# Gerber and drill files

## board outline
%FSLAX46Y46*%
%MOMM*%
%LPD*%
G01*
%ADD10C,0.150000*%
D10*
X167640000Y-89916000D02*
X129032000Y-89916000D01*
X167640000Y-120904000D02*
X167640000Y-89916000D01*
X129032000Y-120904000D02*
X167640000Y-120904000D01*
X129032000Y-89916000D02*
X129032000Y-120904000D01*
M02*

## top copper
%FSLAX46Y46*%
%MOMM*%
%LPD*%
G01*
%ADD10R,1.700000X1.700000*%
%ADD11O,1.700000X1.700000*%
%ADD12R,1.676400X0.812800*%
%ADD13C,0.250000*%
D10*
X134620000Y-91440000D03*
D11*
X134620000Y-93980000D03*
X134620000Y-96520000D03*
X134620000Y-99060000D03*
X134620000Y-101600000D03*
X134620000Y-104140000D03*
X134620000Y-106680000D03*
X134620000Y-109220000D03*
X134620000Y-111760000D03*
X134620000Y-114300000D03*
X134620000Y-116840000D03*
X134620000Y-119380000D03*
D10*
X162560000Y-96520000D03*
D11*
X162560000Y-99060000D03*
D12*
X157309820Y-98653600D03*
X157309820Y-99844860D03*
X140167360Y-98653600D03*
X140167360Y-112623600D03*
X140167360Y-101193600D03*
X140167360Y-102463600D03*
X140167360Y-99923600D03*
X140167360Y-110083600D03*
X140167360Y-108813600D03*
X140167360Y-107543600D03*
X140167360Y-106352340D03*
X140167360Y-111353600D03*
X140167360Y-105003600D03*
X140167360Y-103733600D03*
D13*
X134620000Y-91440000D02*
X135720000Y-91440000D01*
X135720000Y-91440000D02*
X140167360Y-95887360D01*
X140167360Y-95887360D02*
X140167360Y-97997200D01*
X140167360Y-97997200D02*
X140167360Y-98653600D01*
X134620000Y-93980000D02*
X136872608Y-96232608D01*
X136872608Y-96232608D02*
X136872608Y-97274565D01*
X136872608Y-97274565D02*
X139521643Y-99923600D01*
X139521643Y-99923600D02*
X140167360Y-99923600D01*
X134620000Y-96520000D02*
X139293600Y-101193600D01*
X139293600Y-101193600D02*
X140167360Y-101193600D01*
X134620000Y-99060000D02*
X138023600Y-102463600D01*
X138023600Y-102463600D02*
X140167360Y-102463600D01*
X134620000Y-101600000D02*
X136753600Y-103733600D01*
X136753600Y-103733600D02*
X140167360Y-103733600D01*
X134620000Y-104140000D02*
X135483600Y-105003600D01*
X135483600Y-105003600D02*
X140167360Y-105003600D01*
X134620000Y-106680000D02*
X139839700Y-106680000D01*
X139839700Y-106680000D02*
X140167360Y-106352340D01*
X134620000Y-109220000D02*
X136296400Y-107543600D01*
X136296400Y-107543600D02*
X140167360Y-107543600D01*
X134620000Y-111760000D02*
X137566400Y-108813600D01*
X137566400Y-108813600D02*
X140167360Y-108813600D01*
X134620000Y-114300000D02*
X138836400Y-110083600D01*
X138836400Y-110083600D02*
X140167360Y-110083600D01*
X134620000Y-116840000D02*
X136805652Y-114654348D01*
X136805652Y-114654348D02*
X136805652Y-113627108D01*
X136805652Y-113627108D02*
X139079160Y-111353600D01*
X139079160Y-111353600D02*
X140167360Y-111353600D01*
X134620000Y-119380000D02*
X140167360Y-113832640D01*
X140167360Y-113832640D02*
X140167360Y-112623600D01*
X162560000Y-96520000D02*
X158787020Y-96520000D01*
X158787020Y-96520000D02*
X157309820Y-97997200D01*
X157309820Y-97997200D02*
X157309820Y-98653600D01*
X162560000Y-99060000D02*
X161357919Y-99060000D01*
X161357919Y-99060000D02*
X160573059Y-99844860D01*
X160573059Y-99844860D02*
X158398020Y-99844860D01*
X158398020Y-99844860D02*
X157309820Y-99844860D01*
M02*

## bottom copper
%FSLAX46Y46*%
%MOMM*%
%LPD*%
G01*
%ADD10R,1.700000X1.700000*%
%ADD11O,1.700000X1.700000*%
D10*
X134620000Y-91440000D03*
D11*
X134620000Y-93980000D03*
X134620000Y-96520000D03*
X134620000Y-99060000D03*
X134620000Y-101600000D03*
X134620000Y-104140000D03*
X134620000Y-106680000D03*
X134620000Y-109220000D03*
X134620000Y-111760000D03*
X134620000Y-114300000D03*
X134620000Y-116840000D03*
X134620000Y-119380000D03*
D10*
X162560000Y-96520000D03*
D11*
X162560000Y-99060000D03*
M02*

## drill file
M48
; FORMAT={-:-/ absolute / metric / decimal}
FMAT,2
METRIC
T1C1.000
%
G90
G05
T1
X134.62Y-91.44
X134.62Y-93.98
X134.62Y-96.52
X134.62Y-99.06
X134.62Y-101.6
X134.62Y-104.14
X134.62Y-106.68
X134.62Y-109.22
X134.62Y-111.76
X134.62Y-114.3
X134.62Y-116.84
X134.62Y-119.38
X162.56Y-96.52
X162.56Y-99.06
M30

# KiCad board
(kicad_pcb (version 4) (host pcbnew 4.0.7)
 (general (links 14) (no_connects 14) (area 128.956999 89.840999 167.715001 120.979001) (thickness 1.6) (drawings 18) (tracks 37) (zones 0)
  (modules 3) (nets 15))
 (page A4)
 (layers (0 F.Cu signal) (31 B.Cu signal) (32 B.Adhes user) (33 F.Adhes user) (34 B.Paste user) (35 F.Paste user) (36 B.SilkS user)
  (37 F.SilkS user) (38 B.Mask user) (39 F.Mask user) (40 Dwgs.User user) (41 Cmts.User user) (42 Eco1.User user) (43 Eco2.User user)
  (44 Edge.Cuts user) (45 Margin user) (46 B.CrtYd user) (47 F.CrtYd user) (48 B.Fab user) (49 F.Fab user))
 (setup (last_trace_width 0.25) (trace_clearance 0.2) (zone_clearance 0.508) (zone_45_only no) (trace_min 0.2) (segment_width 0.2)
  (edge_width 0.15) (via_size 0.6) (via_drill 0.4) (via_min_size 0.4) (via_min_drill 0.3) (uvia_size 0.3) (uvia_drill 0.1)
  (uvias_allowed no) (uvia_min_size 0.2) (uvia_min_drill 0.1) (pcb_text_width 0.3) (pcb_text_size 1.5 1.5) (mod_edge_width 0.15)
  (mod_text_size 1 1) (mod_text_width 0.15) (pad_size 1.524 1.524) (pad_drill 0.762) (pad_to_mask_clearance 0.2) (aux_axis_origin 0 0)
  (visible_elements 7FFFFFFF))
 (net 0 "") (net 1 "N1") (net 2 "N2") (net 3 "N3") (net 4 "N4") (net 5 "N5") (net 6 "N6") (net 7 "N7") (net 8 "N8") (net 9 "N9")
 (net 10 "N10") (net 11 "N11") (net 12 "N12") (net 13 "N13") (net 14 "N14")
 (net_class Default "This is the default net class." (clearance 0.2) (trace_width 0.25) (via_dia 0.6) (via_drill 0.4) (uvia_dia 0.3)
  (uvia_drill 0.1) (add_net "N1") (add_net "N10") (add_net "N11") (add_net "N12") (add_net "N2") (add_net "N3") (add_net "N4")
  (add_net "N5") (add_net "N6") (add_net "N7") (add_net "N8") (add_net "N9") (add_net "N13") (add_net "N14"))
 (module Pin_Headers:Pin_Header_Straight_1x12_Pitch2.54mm (layer F.Cu) (at 134.62 91.44)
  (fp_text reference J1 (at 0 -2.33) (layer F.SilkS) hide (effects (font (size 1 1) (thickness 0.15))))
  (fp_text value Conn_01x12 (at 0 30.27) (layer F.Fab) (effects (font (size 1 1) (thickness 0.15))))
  (pad 1 thru_hole rect (at 0 0) (size 1.7 1.7) (drill 1) (layers *.Cu *.Mask) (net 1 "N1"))
  (pad 2 thru_hole oval (at 0 2.54) (size 1.7 1.7) (drill 1) (layers *.Cu *.Mask) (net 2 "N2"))
  (pad 3 thru_hole oval (at 0 5.08) (size 1.7 1.7) (drill 1) (layers *.Cu *.Mask) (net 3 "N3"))
  (pad 4 thru_hole oval (at 0 7.62) (size 1.7 1.7) (drill 1) (layers *.Cu *.Mask) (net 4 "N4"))
  (pad 5 thru_hole oval (at 0 10.16) (size 1.7 1.7) (drill 1) (layers *.Cu *.Mask) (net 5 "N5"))
  (pad 6 thru_hole oval (at 0 12.7) (size 1.7 1.7) (drill 1) (layers *.Cu *.Mask) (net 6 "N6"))
  (pad 7 thru_hole oval (at 0 15.24) (size 1.7 1.7) (drill 1) (layers *.Cu *.Mask) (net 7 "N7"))
  (pad 8 thru_hole oval (at 0 17.78) (size 1.7 1.7) (drill 1) (layers *.Cu *.Mask) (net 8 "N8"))
  (pad 9 thru_hole oval (at 0 20.32) (size 1.7 1.7) (drill 1) (layers *.Cu *.Mask) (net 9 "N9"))
  (pad 10 thru_hole oval (at 0 22.86) (size 1.7 1.7) (drill 1) (layers *.Cu *.Mask) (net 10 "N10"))
  (pad 11 thru_hole oval (at 0 25.4) (size 1.7 1.7) (drill 1) (layers *.Cu *.Mask) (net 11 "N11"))
  (pad 12 thru_hole oval (at 0 27.94) (size 1.7 1.7) (drill 1) (layers *.Cu *.Mask) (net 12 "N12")))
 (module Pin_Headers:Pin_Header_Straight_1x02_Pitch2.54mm (layer F.Cu) (at 162.56 96.52)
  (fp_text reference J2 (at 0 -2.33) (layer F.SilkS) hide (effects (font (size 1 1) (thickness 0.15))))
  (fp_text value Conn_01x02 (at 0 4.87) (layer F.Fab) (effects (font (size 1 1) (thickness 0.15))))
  (pad 1 thru_hole rect (at 0 0) (size 1.7 1.7) (drill 1) (layers *.Cu *.Mask) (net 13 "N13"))
  (pad 2 thru_hole oval (at 0 2.54) (size 1.7 1.7) (drill 1) (layers *.Cu *.Mask) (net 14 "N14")))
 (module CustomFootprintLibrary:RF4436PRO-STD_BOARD (layer F.Cu) (at 148.5011 105.0036)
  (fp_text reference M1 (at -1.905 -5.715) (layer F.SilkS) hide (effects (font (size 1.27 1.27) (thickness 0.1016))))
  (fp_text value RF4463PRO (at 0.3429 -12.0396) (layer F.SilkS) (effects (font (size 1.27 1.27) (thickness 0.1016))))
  (pad 13 smd rect (at 8.80872 -6.35) (size 1.6764 0.8128) (layers F.Cu F.Paste F.Mask) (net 13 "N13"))
  (pad 14 smd rect (at 8.80872 -5.15874) (size 1.6764 0.8128) (layers F.Cu F.Paste F.Mask) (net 14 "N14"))
  (pad 1 smd rect (at -8.33374 -6.35) (size 1.6764 0.8128) (layers F.Cu F.Paste F.Mask) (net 1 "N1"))
  (pad 12 smd rect (at -8.33374 7.62) (size 1.6764 0.8128) (layers F.Cu F.Paste F.Mask) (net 12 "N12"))
  (pad 3 smd rect (at -8.33374 -3.81) (size 1.6764 0.8128) (layers F.Cu F.Paste F.Mask) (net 3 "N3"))
  (pad 4 smd rect (at -8.33374 -2.54) (size 1.6764 0.8128) (layers F.Cu F.Paste F.Mask) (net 4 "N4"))
  (pad 2 smd rect (at -8.33374 -5.08) (size 1.6764 0.8128) (layers F.Cu F.Paste F.Mask) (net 2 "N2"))
  (pad 10 smd rect (at -8.33374 5.08) (size 1.6764 0.8128) (layers F.Cu F.Paste F.Mask) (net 10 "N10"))
  (pad 9 smd rect (at -8.33374 3.81) (size 1.6764 0.8128) (layers F.Cu F.Paste F.Mask) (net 9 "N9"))
  (pad 8 smd rect (at -8.33374 2.54) (size 1.6764 0.8128) (layers F.Cu F.Paste F.Mask) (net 8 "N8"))
  (pad 7 smd rect (at -8.33374 1.34874) (size 1.6764 0.8128) (layers F.Cu F.Paste F.Mask) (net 7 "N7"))
  (pad 11 smd rect (at -8.33374 6.35) (size 1.6764 0.8128) (layers F.Cu F.Paste F.Mask) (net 11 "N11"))
  (pad 6 smd rect (at -8.33374 0) (size 1.6764 0.8128) (layers F.Cu F.Paste F.Mask) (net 6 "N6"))
  (pad 5 smd rect (at -8.33374 -1.27) (size 1.6764 0.8128) (layers F.Cu F.Paste F.Mask) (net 5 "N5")))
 (gr_line (start 167.64 89.916) (end 129.032 89.916) (layer Edge.Cuts) (width 0.15))
 (gr_line (start 167.64 120.904) (end 167.64 89.916) (layer Edge.Cuts) (width 0.15))
 (gr_line (start 129.032 120.904) (end 167.64 120.904) (layer Edge.Cuts) (width 0.15))
 (gr_line (start 129.032 89.916) (end 129.032 120.904) (layer Edge.Cuts) (width 0.15))
 (segment (start 134.62 91.44) (end 135.72 91.44) (width 0.25) (layer F.Cu) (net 1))
 (segment (start 135.72 91.44) (end 140.16736 95.88736) (width 0.25) (layer F.Cu) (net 1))
 (segment (start 140.16736 95.88736) (end 140.16736 97.9972) (width 0.25) (layer F.Cu) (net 1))
 (segment (start 140.16736 97.9972) (end 140.16736 98.6536) (width 0.25) (layer F.Cu) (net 1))
 (segment (start 134.62 93.98) (end 136.872608 96.232608) (width 0.25) (layer F.Cu) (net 2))
 (segment (start 136.872608 96.232608) (end 136.872608 97.274565) (width 0.25) (layer F.Cu) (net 2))
 (segment (start 136.872608 97.274565) (end 139.521643 99.9236) (width 0.25) (layer F.Cu) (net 2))
 (segment (start 139.521643 99.9236) (end 140.16736 99.9236) (width 0.25) (layer F.Cu) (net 2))
 (segment (start 134.62 96.52) (end 139.2936 101.1936) (width 0.25) (layer F.Cu) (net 3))
 (segment (start 139.2936 101.1936) (end 140.16736 101.1936) (width 0.25) (layer F.Cu) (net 3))
 (segment (start 134.62 99.06) (end 138.0236 102.4636) (width 0.25) (layer F.Cu) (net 4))
 (segment (start 138.0236 102.4636) (end 140.16736 102.4636) (width 0.25) (layer F.Cu) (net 4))
 (segment (start 134.62 101.6) (end 136.7536 103.7336) (width 0.25) (layer F.Cu) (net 5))
 (segment (start 136.7536 103.7336) (end 140.16736 103.7336) (width 0.25) (layer F.Cu) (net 5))
 (segment (start 134.62 104.14) (end 135.4836 105.0036) (width 0.25) (layer F.Cu) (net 6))
 (segment (start 135.4836 105.0036) (end 140.16736 105.0036) (width 0.25) (layer F.Cu) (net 6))
 (segment (start 134.62 106.68) (end 139.8397 106.68) (width 0.25) (layer F.Cu) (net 7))
 (segment (start 139.8397 106.68) (end 140.16736 106.35234) (width 0.25) (layer F.Cu) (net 7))
 (segment (start 134.62 109.22) (end 136.2964 107.5436) (width 0.25) (layer F.Cu) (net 8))
 (segment (start 136.2964 107.5436) (end 140.16736 107.5436) (width 0.25) (layer F.Cu) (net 8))
 (segment (start 134.62 111.76) (end 137.5664 108.8136) (width 0.25) (layer F.Cu) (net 9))
 (segment (start 137.5664 108.8136) (end 140.16736 108.8136) (width 0.25) (layer F.Cu) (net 9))
 (segment (start 134.62 114.3) (end 138.8364 110.0836) (width 0.25) (layer F.Cu) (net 10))
 (segment (start 138.8364 110.0836) (end 140.16736 110.0836) (width 0.25) (layer F.Cu) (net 10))
 (segment (start 134.62 116.84) (end 136.805652 114.654348) (width 0.25) (layer F.Cu) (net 11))
 (segment (start 136.805652 114.654348) (end 136.805652 113.627108) (width 0.25) (layer F.Cu) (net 11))
 (segment (start 136.805652 113.627108) (end 139.07916 111.3536) (width 0.25) (layer F.Cu) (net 11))
 (segment (start 139.07916 111.3536) (end 140.16736 111.3536) (width 0.25) (layer F.Cu) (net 11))
 (segment (start 134.62 119.38) (end 140.16736 113.83264) (width 0.25) (layer F.Cu) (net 12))
 (segment (start 140.16736 113.83264) (end 140.16736 112.6236) (width 0.25) (layer F.Cu) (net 12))
 (segment (start 162.56 96.52) (end 158.78702 96.52) (width 0.25) (layer F.Cu) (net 13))
 (segment (start 158.78702 96.52) (end 157.30982 97.9972) (width 0.25) (layer F.Cu) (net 13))
 (segment (start 157.30982 97.9972) (end 157.30982 98.6536) (width 0.25) (layer F.Cu) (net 13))
 (segment (start 162.56 99.06) (end 161.357919 99.06) (width 0.25) (layer F.Cu) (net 14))
 (segment (start 161.357919 99.06) (end 160.573059 99.84486) (width 0.25) (layer F.Cu) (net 14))
 (segment (start 160.573059 99.84486) (end 158.39802 99.84486) (width 0.25) (layer F.Cu) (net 14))
 (segment (start 158.39802 99.84486) (end 157.30982 99.84486) (width 0.25) (layer F.Cu) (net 14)))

